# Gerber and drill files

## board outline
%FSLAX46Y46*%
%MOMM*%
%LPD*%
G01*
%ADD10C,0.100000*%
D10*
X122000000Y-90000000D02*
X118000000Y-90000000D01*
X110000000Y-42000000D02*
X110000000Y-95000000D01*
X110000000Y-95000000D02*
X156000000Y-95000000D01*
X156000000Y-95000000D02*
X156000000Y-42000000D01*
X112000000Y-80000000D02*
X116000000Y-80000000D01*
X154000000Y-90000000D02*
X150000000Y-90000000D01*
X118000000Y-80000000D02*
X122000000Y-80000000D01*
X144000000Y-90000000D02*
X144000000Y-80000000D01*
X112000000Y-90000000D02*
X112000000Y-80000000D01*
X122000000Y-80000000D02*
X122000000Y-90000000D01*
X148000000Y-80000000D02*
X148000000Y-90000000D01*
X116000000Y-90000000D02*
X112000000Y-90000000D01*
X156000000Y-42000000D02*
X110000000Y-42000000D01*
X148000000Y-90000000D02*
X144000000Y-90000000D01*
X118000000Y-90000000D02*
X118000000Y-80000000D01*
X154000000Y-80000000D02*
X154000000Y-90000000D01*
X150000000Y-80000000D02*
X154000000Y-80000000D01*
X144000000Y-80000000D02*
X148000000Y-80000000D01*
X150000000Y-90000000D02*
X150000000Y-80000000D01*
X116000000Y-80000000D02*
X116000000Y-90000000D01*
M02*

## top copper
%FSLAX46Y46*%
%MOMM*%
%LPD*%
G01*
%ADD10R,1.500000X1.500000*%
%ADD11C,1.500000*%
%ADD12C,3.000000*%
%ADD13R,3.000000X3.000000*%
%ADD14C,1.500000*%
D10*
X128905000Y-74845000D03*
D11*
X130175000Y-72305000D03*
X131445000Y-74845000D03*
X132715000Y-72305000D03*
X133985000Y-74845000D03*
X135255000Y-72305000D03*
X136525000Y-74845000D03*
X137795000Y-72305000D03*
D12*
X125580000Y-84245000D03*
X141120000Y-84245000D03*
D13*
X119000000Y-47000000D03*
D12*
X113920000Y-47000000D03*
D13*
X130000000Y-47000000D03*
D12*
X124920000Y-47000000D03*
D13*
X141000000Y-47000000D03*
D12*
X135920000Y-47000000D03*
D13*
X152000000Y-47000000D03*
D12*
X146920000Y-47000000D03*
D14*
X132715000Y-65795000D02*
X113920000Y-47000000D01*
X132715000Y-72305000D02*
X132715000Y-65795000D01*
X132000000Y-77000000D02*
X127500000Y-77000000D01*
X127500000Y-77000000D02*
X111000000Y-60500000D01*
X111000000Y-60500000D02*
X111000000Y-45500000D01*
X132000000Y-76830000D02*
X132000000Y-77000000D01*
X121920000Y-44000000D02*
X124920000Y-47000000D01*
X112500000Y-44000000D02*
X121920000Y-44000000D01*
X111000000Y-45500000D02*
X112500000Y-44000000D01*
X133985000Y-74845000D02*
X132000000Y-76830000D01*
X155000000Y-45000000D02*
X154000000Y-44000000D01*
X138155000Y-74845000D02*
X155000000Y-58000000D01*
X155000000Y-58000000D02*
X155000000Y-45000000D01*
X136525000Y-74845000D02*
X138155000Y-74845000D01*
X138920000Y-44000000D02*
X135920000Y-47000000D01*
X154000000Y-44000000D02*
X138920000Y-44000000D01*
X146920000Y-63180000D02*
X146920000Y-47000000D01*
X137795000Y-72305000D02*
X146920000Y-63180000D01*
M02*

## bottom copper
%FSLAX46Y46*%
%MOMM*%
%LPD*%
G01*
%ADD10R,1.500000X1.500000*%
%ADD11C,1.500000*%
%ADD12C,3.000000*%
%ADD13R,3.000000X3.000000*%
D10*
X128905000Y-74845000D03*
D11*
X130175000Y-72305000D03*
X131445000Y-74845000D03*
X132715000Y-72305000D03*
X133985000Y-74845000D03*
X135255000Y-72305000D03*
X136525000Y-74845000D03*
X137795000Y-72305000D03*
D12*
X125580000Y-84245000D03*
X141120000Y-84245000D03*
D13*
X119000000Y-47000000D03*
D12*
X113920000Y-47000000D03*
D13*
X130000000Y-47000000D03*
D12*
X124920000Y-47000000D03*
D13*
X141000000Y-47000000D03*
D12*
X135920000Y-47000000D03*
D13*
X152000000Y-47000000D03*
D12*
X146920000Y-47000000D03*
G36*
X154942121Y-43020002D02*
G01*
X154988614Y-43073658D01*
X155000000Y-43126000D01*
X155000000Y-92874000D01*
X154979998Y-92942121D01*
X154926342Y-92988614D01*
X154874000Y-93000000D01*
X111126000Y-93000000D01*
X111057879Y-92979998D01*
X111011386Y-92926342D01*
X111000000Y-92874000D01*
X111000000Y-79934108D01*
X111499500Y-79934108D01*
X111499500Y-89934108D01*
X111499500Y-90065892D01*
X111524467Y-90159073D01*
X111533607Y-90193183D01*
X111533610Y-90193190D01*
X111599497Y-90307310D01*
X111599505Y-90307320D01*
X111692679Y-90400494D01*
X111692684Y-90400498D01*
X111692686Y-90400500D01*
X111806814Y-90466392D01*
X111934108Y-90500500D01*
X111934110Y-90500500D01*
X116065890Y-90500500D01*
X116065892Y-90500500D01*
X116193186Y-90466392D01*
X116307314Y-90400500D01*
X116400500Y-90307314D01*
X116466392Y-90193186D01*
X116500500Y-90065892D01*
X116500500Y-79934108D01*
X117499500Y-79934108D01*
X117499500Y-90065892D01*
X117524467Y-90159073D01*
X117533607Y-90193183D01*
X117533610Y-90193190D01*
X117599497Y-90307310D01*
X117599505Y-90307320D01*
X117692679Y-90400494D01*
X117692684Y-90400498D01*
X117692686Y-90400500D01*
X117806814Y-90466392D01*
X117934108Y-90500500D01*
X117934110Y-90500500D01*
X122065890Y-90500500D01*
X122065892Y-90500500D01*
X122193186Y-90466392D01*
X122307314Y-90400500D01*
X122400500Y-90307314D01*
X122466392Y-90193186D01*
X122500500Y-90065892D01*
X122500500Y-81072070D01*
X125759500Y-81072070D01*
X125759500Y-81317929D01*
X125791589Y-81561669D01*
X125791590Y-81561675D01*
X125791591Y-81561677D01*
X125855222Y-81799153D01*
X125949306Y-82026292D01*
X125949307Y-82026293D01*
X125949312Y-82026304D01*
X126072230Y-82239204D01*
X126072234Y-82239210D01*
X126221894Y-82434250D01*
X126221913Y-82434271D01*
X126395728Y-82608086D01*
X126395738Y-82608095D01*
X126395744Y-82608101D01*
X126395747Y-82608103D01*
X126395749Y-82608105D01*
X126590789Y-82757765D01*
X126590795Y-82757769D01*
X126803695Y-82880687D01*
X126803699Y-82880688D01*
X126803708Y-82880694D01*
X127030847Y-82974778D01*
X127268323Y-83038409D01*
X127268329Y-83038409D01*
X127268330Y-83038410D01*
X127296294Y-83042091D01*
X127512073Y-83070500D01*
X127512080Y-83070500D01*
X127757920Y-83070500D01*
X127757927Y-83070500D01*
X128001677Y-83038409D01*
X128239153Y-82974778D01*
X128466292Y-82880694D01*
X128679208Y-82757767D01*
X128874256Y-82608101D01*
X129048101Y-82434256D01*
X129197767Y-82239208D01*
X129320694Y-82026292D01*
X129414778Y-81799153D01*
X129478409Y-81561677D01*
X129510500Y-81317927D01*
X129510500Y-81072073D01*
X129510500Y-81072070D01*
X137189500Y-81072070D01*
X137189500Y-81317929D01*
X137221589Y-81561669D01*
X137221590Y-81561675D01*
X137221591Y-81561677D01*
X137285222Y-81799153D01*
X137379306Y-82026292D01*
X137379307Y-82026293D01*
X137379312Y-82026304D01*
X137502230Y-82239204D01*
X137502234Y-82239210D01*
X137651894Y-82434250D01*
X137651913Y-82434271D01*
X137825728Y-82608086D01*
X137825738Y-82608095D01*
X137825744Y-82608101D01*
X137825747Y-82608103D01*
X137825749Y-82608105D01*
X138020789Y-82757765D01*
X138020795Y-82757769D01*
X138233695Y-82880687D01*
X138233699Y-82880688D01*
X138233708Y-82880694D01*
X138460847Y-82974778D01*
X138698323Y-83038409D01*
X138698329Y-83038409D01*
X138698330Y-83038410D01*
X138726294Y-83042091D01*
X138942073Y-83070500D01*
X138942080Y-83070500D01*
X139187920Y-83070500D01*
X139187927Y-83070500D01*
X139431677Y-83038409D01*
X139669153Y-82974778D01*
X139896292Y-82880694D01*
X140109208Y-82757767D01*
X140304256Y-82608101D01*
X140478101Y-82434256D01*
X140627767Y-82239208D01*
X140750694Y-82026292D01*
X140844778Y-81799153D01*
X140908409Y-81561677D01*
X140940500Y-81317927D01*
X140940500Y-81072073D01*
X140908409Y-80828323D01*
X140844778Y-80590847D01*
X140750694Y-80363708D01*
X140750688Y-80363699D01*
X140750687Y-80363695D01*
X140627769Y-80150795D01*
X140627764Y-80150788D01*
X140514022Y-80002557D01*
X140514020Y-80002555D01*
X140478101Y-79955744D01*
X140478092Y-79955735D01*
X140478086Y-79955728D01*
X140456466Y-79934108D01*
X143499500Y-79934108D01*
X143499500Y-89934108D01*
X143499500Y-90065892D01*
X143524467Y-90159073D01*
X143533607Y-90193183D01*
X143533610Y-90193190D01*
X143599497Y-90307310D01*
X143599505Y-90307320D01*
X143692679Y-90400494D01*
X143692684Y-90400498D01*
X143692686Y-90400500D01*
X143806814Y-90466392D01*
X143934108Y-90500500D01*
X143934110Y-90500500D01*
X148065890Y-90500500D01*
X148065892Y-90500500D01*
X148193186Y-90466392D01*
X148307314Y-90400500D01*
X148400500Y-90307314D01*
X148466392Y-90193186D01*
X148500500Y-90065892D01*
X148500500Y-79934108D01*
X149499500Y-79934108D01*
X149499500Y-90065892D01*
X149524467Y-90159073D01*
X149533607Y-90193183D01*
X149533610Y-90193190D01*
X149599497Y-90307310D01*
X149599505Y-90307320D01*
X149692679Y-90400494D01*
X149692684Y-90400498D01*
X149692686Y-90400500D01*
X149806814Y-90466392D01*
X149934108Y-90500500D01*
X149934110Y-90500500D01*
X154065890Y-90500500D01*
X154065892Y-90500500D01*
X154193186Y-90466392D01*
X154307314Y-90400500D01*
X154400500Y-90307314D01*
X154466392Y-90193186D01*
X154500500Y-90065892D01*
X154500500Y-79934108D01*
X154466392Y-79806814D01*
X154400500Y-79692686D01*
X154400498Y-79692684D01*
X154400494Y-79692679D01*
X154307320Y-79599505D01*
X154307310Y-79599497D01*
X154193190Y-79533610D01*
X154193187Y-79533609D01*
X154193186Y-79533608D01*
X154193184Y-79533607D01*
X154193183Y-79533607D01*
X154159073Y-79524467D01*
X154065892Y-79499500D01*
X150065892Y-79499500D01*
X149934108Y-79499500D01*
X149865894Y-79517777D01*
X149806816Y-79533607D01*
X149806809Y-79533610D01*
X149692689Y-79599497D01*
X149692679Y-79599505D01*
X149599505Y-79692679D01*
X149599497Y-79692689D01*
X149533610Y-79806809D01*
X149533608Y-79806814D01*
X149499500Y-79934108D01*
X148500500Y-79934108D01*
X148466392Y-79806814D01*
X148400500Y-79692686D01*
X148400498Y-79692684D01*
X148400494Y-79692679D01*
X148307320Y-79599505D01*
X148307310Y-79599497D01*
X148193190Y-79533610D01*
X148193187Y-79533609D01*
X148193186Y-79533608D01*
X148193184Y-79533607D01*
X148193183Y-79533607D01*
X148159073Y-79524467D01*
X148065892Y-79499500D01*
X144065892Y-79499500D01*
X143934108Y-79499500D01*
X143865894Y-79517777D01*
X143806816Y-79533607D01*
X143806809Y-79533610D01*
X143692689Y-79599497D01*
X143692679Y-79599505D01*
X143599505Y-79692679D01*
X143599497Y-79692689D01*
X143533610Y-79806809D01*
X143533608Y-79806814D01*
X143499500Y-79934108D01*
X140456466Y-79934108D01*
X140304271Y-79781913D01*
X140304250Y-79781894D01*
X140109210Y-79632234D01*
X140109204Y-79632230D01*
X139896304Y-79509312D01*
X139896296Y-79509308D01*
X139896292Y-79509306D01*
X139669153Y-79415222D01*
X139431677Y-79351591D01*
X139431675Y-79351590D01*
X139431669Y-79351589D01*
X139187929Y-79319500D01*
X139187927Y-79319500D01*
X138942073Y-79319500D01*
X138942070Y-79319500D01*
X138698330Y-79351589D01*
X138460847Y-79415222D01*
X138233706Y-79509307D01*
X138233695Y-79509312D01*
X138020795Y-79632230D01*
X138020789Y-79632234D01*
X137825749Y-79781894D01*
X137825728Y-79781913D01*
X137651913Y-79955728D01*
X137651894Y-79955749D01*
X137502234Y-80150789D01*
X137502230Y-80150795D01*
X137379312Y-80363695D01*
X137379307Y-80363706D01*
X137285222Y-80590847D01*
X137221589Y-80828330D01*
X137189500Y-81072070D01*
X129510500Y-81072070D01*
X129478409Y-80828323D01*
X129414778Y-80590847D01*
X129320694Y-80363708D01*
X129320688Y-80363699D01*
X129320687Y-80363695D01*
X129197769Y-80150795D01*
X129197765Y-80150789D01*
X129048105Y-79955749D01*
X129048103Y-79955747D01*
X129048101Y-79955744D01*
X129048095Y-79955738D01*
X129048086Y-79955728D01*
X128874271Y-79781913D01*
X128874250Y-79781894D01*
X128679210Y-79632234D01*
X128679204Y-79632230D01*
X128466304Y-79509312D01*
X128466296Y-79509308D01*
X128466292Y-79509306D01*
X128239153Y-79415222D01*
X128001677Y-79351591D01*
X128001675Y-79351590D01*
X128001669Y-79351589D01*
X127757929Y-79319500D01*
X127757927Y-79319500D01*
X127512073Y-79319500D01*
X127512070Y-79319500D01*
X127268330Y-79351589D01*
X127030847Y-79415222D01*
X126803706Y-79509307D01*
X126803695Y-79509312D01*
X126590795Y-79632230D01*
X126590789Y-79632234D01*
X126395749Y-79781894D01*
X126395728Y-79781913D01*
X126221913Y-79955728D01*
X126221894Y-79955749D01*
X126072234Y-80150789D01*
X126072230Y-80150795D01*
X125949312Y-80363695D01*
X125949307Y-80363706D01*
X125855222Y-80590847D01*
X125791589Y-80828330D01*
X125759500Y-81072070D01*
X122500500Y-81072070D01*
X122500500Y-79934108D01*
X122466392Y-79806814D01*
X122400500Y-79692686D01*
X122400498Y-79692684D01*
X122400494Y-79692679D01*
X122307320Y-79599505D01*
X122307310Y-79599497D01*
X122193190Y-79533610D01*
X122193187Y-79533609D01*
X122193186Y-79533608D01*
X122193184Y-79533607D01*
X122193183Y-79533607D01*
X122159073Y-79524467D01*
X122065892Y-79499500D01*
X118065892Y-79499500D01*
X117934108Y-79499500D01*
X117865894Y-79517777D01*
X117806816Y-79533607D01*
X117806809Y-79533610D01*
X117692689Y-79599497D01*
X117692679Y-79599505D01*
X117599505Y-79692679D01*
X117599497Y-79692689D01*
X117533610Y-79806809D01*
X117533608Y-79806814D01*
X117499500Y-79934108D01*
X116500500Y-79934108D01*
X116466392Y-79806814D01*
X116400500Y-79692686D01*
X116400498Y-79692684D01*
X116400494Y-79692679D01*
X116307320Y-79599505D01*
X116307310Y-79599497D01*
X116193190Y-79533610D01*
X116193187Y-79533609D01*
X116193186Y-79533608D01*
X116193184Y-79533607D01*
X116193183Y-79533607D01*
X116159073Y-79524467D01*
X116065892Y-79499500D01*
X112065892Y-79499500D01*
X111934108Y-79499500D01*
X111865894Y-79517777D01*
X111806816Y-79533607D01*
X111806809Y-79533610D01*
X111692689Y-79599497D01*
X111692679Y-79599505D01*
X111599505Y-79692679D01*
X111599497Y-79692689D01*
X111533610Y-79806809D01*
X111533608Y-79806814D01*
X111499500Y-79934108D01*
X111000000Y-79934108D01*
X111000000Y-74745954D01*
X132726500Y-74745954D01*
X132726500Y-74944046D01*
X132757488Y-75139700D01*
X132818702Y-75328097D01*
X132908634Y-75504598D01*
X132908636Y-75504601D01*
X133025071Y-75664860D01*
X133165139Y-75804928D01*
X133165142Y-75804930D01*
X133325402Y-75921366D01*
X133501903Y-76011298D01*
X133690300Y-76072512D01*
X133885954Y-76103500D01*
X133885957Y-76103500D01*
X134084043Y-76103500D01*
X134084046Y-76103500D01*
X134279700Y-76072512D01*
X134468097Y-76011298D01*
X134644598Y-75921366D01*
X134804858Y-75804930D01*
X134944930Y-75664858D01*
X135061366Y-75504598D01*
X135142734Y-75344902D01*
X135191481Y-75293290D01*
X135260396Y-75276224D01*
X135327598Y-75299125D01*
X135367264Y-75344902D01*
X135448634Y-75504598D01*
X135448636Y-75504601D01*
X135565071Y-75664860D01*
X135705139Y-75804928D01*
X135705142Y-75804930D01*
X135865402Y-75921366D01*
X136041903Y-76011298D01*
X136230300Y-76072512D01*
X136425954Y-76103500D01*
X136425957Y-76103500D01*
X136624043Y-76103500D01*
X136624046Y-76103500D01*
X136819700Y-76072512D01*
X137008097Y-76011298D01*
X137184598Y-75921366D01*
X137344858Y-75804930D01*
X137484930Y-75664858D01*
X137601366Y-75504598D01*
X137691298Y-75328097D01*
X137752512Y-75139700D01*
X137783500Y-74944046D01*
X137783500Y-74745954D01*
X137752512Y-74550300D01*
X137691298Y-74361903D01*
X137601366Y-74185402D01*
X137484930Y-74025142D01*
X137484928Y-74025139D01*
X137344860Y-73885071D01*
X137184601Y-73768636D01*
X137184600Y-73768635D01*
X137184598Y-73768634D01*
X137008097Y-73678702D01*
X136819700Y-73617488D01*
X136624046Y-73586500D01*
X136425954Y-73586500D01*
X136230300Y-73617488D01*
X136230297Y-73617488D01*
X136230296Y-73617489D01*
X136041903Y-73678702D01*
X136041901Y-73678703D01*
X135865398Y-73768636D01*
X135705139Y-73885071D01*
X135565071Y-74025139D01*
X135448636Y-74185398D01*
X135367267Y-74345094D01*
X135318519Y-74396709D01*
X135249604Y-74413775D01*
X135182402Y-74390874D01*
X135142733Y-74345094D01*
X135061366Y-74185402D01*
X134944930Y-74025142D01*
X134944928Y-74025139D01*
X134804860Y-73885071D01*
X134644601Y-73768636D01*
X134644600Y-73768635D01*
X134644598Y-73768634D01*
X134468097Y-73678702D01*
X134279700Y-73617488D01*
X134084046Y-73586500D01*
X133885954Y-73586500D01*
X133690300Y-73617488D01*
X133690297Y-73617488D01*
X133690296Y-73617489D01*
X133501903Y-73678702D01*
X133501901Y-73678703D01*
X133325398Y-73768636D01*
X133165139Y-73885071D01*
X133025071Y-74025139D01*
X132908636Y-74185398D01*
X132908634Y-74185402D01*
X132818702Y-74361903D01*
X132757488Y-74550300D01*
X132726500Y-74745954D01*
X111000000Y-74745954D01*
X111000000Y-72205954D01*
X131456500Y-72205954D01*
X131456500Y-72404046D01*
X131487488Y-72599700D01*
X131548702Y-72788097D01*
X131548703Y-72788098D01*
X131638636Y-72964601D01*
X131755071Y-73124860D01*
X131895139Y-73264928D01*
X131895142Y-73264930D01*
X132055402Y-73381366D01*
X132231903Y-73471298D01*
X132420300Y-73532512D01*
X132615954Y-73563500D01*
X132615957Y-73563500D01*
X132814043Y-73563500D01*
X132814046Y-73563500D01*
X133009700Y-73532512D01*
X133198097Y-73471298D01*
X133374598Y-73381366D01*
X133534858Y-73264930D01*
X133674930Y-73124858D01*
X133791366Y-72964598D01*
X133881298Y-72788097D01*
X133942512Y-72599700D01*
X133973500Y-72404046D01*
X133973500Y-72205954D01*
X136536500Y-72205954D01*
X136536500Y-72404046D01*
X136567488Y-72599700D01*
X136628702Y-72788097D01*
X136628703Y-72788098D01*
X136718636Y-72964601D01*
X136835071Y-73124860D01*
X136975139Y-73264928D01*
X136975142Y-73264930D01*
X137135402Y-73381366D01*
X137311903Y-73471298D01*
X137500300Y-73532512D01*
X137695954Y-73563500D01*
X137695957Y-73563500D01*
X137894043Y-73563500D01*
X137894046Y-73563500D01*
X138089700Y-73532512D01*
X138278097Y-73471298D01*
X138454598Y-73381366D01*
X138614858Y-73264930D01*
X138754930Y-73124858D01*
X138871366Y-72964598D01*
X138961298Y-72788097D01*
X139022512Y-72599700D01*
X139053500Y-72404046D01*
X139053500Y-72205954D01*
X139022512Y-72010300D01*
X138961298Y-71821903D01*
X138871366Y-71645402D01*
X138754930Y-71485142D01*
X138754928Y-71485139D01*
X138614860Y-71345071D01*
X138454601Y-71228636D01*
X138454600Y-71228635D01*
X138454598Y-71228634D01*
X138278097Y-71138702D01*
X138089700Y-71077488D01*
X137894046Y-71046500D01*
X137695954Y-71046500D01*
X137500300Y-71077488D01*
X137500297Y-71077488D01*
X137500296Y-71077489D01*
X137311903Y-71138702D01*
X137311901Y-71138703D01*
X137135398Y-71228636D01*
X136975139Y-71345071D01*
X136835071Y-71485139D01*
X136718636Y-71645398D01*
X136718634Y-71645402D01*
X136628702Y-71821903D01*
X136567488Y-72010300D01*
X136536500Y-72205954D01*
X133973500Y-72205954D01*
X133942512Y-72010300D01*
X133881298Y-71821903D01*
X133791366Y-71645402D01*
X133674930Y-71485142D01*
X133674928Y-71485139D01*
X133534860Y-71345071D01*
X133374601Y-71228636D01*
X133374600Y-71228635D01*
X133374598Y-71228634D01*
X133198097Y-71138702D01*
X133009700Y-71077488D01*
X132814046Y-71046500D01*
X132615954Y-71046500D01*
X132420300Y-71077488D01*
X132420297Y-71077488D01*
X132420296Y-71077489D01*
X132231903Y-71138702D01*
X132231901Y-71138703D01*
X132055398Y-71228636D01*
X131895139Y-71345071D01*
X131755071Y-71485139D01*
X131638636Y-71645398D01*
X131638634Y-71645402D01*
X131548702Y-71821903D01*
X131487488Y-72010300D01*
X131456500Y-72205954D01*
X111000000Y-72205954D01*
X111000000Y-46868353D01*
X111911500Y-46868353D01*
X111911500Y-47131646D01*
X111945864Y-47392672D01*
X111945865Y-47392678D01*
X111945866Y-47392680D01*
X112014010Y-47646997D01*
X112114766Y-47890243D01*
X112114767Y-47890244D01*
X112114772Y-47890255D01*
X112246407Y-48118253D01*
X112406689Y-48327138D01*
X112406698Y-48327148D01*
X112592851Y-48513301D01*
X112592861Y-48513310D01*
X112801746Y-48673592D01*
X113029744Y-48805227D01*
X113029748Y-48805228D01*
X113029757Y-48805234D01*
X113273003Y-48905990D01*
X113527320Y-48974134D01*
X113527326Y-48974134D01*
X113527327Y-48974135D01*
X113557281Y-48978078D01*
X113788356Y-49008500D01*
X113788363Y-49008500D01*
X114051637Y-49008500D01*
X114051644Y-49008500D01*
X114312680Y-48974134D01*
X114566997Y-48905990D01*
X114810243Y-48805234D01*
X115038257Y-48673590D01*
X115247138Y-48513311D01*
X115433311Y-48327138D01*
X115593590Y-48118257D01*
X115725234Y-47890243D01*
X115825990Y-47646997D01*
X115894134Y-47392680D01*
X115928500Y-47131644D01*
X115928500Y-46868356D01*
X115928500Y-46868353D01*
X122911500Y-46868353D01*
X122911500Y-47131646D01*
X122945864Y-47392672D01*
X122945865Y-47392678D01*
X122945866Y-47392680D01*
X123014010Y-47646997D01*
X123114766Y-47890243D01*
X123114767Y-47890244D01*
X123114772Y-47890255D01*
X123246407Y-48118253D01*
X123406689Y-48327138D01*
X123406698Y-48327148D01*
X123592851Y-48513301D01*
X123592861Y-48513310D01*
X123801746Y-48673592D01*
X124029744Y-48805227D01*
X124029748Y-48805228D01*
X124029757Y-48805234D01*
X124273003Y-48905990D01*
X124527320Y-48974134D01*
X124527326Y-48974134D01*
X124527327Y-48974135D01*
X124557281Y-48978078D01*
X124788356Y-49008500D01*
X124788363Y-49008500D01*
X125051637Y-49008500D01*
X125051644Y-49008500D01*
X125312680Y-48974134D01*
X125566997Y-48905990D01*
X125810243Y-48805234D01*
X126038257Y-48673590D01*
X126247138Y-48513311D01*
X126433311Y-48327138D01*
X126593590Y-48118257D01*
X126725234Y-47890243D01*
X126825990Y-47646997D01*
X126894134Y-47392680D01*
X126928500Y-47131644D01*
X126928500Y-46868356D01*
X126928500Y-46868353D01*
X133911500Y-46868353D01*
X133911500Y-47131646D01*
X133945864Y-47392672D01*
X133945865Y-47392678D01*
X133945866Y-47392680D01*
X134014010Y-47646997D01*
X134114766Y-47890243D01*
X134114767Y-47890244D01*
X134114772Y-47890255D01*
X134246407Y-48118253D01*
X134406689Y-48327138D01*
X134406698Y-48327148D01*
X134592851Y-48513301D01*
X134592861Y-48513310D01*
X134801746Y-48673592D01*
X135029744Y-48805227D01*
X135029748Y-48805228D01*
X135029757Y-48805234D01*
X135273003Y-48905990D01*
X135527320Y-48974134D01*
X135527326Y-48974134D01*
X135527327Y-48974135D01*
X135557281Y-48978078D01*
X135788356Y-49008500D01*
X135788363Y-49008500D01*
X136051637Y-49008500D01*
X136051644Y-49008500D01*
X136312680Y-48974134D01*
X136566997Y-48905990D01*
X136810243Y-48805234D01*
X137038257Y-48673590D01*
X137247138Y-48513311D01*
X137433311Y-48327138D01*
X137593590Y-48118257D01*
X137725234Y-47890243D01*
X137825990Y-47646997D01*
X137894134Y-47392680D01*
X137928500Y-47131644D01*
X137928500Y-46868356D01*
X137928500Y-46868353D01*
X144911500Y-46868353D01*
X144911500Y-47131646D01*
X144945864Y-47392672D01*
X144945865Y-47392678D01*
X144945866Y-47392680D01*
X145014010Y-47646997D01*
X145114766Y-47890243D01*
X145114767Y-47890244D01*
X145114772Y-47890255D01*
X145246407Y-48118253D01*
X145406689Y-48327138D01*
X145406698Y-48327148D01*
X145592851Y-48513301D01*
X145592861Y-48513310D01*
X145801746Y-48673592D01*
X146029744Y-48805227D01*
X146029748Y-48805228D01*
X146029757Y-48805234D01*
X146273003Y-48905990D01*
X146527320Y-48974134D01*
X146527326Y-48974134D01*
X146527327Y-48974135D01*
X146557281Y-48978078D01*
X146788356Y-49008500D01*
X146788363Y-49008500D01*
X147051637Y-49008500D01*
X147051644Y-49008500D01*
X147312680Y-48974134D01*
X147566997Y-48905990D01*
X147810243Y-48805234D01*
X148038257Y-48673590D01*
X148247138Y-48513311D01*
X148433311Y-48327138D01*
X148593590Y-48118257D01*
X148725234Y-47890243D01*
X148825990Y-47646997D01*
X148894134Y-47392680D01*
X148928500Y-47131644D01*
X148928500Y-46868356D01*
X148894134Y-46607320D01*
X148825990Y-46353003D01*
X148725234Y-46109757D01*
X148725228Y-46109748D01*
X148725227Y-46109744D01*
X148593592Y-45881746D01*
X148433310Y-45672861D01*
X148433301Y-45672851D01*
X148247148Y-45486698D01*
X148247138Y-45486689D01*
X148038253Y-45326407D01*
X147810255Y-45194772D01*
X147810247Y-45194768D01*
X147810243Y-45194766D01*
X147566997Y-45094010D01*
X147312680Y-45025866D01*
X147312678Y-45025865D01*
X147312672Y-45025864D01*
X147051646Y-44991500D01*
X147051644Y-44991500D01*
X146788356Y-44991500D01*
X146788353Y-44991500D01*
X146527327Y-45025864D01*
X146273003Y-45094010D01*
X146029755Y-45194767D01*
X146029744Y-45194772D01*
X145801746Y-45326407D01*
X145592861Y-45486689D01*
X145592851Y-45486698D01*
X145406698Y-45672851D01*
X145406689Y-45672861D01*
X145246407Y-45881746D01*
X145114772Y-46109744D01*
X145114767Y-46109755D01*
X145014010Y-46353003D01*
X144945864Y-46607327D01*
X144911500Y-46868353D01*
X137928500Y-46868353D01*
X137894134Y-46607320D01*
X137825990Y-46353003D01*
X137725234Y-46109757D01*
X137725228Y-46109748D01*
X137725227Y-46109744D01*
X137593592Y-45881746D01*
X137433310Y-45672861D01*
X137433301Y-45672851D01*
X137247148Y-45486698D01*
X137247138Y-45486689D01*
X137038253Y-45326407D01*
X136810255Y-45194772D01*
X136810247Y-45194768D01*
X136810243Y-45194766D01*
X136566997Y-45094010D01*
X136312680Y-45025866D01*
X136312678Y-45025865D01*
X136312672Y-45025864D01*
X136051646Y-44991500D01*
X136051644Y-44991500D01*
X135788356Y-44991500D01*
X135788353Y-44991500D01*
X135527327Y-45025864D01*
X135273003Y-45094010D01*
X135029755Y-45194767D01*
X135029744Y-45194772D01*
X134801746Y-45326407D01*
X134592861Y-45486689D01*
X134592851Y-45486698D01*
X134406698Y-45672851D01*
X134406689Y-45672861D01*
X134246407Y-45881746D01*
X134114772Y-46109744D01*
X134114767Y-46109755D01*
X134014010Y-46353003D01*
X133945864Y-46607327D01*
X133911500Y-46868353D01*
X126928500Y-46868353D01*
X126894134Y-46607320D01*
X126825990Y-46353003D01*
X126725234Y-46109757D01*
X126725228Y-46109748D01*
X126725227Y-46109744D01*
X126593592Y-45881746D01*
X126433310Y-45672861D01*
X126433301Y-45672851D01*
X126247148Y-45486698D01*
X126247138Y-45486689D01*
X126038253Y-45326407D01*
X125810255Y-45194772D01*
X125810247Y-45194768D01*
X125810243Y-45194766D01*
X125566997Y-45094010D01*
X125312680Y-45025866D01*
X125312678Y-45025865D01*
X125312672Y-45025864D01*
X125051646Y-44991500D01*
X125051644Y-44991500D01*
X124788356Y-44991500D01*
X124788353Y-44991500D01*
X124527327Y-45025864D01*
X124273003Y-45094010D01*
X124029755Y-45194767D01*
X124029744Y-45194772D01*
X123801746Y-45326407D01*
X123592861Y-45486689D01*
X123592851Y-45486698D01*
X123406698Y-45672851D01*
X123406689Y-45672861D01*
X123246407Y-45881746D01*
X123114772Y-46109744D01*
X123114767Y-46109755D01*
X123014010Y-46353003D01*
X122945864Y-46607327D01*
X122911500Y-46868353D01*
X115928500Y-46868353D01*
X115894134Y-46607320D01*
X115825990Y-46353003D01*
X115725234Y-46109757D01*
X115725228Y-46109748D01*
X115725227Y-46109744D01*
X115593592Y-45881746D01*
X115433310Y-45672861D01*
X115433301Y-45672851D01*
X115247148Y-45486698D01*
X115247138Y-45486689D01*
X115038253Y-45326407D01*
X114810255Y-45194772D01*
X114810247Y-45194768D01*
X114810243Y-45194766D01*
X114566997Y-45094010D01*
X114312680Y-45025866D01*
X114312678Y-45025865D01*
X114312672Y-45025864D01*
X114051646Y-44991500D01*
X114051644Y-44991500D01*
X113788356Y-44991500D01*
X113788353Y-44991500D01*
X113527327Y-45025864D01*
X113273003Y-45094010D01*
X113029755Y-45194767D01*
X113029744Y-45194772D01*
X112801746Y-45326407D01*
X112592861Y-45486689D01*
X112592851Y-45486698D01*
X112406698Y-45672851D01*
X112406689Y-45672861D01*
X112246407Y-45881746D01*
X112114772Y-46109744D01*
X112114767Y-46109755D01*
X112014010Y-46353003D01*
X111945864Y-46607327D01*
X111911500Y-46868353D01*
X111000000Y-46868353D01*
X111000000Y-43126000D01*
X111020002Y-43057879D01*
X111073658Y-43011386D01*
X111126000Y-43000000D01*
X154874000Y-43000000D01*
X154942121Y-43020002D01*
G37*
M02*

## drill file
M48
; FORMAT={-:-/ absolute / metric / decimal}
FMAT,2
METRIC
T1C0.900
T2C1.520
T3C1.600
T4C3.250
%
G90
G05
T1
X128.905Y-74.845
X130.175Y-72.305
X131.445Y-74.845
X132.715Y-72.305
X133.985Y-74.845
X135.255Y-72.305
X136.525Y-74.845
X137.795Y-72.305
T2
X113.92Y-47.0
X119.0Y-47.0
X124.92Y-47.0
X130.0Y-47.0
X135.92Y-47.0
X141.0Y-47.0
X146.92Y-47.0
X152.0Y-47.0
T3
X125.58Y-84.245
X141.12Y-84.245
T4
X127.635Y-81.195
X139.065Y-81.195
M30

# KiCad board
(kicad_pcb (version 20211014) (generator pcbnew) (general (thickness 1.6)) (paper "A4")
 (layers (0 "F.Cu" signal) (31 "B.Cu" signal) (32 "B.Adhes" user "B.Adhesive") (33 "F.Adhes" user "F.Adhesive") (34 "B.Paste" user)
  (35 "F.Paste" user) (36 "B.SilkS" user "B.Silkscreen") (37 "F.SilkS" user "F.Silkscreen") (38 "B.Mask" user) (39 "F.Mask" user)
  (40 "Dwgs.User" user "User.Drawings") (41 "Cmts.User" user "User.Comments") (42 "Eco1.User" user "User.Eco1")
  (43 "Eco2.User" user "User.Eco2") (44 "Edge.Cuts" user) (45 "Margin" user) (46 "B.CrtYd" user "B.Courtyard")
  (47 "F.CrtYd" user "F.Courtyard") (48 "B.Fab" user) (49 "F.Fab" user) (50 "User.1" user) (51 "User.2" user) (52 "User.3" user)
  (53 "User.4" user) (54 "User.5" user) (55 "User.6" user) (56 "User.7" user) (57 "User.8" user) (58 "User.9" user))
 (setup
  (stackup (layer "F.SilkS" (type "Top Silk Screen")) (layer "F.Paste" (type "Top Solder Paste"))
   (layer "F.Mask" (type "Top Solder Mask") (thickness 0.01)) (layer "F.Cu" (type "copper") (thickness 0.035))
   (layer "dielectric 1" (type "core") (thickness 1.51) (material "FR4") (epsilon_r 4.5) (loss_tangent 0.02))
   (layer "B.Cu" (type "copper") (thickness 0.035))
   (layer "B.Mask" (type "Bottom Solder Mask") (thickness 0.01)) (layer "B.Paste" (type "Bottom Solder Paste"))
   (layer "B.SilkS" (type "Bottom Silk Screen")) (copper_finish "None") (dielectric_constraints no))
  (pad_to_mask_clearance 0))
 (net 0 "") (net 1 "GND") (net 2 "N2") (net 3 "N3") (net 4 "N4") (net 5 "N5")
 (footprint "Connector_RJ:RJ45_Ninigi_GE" (layer "F.Cu") (at 128.905 74.845)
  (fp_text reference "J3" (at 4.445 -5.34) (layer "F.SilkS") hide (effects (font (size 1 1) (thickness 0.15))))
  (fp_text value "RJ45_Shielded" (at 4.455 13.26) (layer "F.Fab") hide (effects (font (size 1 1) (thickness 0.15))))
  (pad "" np_thru_hole circle (at -1.27 6.35) (size 3.25 3.25) (drill 3.25) (layers *.Cu *.Mask))
  (pad "" np_thru_hole circle (at 10.16 6.35 180) (size 3.25 3.25) (drill 3.25) (layers *.Cu *.Mask))
  (pad "1" thru_hole rect (at 0 0 180) (size 1.5 1.5) (drill 0.9) (layers *.Cu *.Mask) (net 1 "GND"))
  (pad "2" thru_hole circle (at 1.27 -2.54 180) (size 1.5 1.5) (drill 0.9) (layers *.Cu *.Mask) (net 1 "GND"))
  (pad "3" thru_hole circle (at 2.54 0 180) (size 1.5 1.5) (drill 0.9) (layers *.Cu *.Mask) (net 1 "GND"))
  (pad "4" thru_hole circle (at 3.81 -2.54 180) (size 1.5 1.5) (drill 0.9) (layers *.Cu *.Mask) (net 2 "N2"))
  (pad "5" thru_hole circle (at 5.08 0 180) (size 1.5 1.5) (drill 0.9) (layers *.Cu *.Mask) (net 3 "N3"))
  (pad "6" thru_hole circle (at 6.35 -2.54 180) (size 1.5 1.5) (drill 0.9) (layers *.Cu *.Mask) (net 1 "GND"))
  (pad "7" thru_hole circle (at 7.62 0 180) (size 1.5 1.5) (drill 0.9) (layers *.Cu *.Mask) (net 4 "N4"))
  (pad "8" thru_hole circle (at 8.89 -2.54 180) (size 1.5 1.5) (drill 0.9) (layers *.Cu *.Mask) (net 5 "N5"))
  (pad "SH" thru_hole circle (at -3.325 9.4) (size 3 3) (drill 1.6) (layers *.Cu *.Mask) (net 1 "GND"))
  (pad "SH" thru_hole circle (at 12.215 9.4 180) (size 3 3) (drill 1.6) (layers *.Cu *.Mask) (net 1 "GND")))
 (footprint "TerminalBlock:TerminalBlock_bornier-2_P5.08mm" (layer "F.Cu") (at 119 47 180)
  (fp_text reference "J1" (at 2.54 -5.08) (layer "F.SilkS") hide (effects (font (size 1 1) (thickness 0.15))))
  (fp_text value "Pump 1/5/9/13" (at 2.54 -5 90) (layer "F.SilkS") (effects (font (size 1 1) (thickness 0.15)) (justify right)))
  (pad "1" thru_hole rect (at 0 0 180) (size 3 3) (drill 1.52) (layers *.Cu *.Mask) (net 1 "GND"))
  (pad "2" thru_hole circle (at 5.08 0 180) (size 3 3) (drill 1.52) (layers *.Cu *.Mask) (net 2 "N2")))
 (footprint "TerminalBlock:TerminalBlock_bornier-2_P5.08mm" (layer "F.Cu") (at 130 47 180)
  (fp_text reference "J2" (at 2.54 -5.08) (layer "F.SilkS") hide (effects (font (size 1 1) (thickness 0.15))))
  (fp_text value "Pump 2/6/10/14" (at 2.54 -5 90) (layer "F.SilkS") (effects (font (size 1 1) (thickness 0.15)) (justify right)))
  (pad "1" thru_hole rect (at 0 0 180) (size 3 3) (drill 1.52) (layers *.Cu *.Mask) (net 1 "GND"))
  (pad "2" thru_hole circle (at 5.08 0 180) (size 3 3) (drill 1.52) (layers *.Cu *.Mask) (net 3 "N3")))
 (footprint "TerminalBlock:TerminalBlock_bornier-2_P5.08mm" (layer "F.Cu") (at 141 47 180)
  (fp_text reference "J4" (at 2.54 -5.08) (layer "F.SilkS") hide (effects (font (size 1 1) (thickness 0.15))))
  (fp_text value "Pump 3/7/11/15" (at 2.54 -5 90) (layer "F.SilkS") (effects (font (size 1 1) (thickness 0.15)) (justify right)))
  (pad "1" thru_hole rect (at 0 0 180) (size 3 3) (drill 1.52) (layers *.Cu *.Mask) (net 1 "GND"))
  (pad "2" thru_hole circle (at 5.08 0 180) (size 3 3) (drill 1.52) (layers *.Cu *.Mask) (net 4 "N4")))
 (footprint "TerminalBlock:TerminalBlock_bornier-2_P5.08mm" (layer "F.Cu") (at 152 47 180)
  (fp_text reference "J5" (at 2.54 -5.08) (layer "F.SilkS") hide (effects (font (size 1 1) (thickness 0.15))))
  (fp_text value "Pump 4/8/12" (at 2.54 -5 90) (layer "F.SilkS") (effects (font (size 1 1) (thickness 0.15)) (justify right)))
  (pad "1" thru_hole rect (at 0 0 180) (size 3 3) (drill 1.52) (layers *.Cu *.Mask) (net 1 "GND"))
  (pad "2" thru_hole circle (at 5.08 0 180) (size 3 3) (drill 1.52) (layers *.Cu *.Mask) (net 5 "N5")))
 (gr_line (start 122 90) (end 118 90) (layer "Edge.Cuts") (width 0.1))
 (gr_line (start 110 42) (end 110 95) (layer "Edge.Cuts") (width 0.1))
 (gr_line (start 110 95) (end 156 95) (layer "Edge.Cuts") (width 0.1))
 (gr_line (start 156 95) (end 156 42) (layer "Edge.Cuts") (width 0.1))
 (gr_line (start 112 80) (end 116 80) (layer "Edge.Cuts") (width 0.1))
 (gr_line (start 154 90) (end 150 90) (layer "Edge.Cuts") (width 0.1))
 (gr_line (start 118 80) (end 122 80) (layer "Edge.Cuts") (width 0.1))
 (gr_line (start 144 90) (end 144 80) (layer "Edge.Cuts") (width 0.1))
 (gr_line (start 112 90) (end 112 80) (layer "Edge.Cuts") (width 0.1))
 (gr_line (start 122 80) (end 122 90) (layer "Edge.Cuts") (width 0.1))
 (gr_line (start 148 80) (end 148 90) (layer "Edge.Cuts") (width 0.1))
 (gr_line (start 116 90) (end 112 90) (layer "Edge.Cuts") (width 0.1))
 (gr_line (start 156 42) (end 110 42) (layer "Edge.Cuts") (width 0.1))
 (gr_line (start 148 90) (end 144 90) (layer "Edge.Cuts") (width 0.1))
 (gr_line (start 118 90) (end 118 80) (layer "Edge.Cuts") (width 0.1))
 (gr_line (start 154 80) (end 154 90) (layer "Edge.Cuts") (width 0.1))
 (gr_line (start 150 80) (end 154 80) (layer "Edge.Cuts") (width 0.1))
 (gr_line (start 144 80) (end 148 80) (layer "Edge.Cuts") (width 0.1))
 (gr_line (start 150 90) (end 150 80) (layer "Edge.Cuts") (width 0.1))
 (gr_line (start 116 80) (end 116 90) (layer "Edge.Cuts") (width 0.1))
 (segment (start 132.715 65.795) (end 113.92 47) (width 1.5) (layer "F.Cu") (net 2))
 (segment (start 132.715 72.305) (end 132.715 65.795) (width 1.5) (layer "F.Cu") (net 2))
 (segment (start 132 77) (end 127.5 77) (width 1.5) (layer "F.Cu") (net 3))
 (segment (start 127.5 77) (end 111 60.5) (width 1.5) (layer "F.Cu") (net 3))
 (segment (start 111 60.5) (end 111 45.5) (width 1.5) (layer "F.Cu") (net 3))
 (segment (start 132 76.83) (end 132 77) (width 1.5) (layer "F.Cu") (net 3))
 (segment (start 121.92 44) (end 124.92 47) (width 1.5) (layer "F.Cu") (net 3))
 (segment (start 112.5 44) (end 121.92 44) (width 1.5) (layer "F.Cu") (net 3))
 (segment (start 111 45.5) (end 112.5 44) (width 1.5) (layer "F.Cu") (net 3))
 (segment (start 133.985 74.845) (end 132 76.83) (width 1.5) (layer "F.Cu") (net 3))
 (segment (start 155 45) (end 154 44) (width 1.5) (layer "F.Cu") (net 4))
 (segment (start 138.155 74.845) (end 155 58) (width 1.5) (layer "F.Cu") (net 4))
 (segment (start 155 58) (end 155 45) (width 1.5) (layer "F.Cu") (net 4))
 (segment (start 136.525 74.845) (end 138.155 74.845) (width 1.5) (layer "F.Cu") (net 4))
 (segment (start 138.92 44) (end 135.92 47) (width 1.5) (layer "F.Cu") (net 4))
 (segment (start 154 44) (end 138.92 44) (width 1.5) (layer "F.Cu") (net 4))
 (segment (start 146.92 63.18) (end 146.92 47) (width 1.5) (layer "F.Cu") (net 5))
 (segment (start 137.795 72.305) (end 146.92 63.18) (width 1.5) (layer "F.Cu") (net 5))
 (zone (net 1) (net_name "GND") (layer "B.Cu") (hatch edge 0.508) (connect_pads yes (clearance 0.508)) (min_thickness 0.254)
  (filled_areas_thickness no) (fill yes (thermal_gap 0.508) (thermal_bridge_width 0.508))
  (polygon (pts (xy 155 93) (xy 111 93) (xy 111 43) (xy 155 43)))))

